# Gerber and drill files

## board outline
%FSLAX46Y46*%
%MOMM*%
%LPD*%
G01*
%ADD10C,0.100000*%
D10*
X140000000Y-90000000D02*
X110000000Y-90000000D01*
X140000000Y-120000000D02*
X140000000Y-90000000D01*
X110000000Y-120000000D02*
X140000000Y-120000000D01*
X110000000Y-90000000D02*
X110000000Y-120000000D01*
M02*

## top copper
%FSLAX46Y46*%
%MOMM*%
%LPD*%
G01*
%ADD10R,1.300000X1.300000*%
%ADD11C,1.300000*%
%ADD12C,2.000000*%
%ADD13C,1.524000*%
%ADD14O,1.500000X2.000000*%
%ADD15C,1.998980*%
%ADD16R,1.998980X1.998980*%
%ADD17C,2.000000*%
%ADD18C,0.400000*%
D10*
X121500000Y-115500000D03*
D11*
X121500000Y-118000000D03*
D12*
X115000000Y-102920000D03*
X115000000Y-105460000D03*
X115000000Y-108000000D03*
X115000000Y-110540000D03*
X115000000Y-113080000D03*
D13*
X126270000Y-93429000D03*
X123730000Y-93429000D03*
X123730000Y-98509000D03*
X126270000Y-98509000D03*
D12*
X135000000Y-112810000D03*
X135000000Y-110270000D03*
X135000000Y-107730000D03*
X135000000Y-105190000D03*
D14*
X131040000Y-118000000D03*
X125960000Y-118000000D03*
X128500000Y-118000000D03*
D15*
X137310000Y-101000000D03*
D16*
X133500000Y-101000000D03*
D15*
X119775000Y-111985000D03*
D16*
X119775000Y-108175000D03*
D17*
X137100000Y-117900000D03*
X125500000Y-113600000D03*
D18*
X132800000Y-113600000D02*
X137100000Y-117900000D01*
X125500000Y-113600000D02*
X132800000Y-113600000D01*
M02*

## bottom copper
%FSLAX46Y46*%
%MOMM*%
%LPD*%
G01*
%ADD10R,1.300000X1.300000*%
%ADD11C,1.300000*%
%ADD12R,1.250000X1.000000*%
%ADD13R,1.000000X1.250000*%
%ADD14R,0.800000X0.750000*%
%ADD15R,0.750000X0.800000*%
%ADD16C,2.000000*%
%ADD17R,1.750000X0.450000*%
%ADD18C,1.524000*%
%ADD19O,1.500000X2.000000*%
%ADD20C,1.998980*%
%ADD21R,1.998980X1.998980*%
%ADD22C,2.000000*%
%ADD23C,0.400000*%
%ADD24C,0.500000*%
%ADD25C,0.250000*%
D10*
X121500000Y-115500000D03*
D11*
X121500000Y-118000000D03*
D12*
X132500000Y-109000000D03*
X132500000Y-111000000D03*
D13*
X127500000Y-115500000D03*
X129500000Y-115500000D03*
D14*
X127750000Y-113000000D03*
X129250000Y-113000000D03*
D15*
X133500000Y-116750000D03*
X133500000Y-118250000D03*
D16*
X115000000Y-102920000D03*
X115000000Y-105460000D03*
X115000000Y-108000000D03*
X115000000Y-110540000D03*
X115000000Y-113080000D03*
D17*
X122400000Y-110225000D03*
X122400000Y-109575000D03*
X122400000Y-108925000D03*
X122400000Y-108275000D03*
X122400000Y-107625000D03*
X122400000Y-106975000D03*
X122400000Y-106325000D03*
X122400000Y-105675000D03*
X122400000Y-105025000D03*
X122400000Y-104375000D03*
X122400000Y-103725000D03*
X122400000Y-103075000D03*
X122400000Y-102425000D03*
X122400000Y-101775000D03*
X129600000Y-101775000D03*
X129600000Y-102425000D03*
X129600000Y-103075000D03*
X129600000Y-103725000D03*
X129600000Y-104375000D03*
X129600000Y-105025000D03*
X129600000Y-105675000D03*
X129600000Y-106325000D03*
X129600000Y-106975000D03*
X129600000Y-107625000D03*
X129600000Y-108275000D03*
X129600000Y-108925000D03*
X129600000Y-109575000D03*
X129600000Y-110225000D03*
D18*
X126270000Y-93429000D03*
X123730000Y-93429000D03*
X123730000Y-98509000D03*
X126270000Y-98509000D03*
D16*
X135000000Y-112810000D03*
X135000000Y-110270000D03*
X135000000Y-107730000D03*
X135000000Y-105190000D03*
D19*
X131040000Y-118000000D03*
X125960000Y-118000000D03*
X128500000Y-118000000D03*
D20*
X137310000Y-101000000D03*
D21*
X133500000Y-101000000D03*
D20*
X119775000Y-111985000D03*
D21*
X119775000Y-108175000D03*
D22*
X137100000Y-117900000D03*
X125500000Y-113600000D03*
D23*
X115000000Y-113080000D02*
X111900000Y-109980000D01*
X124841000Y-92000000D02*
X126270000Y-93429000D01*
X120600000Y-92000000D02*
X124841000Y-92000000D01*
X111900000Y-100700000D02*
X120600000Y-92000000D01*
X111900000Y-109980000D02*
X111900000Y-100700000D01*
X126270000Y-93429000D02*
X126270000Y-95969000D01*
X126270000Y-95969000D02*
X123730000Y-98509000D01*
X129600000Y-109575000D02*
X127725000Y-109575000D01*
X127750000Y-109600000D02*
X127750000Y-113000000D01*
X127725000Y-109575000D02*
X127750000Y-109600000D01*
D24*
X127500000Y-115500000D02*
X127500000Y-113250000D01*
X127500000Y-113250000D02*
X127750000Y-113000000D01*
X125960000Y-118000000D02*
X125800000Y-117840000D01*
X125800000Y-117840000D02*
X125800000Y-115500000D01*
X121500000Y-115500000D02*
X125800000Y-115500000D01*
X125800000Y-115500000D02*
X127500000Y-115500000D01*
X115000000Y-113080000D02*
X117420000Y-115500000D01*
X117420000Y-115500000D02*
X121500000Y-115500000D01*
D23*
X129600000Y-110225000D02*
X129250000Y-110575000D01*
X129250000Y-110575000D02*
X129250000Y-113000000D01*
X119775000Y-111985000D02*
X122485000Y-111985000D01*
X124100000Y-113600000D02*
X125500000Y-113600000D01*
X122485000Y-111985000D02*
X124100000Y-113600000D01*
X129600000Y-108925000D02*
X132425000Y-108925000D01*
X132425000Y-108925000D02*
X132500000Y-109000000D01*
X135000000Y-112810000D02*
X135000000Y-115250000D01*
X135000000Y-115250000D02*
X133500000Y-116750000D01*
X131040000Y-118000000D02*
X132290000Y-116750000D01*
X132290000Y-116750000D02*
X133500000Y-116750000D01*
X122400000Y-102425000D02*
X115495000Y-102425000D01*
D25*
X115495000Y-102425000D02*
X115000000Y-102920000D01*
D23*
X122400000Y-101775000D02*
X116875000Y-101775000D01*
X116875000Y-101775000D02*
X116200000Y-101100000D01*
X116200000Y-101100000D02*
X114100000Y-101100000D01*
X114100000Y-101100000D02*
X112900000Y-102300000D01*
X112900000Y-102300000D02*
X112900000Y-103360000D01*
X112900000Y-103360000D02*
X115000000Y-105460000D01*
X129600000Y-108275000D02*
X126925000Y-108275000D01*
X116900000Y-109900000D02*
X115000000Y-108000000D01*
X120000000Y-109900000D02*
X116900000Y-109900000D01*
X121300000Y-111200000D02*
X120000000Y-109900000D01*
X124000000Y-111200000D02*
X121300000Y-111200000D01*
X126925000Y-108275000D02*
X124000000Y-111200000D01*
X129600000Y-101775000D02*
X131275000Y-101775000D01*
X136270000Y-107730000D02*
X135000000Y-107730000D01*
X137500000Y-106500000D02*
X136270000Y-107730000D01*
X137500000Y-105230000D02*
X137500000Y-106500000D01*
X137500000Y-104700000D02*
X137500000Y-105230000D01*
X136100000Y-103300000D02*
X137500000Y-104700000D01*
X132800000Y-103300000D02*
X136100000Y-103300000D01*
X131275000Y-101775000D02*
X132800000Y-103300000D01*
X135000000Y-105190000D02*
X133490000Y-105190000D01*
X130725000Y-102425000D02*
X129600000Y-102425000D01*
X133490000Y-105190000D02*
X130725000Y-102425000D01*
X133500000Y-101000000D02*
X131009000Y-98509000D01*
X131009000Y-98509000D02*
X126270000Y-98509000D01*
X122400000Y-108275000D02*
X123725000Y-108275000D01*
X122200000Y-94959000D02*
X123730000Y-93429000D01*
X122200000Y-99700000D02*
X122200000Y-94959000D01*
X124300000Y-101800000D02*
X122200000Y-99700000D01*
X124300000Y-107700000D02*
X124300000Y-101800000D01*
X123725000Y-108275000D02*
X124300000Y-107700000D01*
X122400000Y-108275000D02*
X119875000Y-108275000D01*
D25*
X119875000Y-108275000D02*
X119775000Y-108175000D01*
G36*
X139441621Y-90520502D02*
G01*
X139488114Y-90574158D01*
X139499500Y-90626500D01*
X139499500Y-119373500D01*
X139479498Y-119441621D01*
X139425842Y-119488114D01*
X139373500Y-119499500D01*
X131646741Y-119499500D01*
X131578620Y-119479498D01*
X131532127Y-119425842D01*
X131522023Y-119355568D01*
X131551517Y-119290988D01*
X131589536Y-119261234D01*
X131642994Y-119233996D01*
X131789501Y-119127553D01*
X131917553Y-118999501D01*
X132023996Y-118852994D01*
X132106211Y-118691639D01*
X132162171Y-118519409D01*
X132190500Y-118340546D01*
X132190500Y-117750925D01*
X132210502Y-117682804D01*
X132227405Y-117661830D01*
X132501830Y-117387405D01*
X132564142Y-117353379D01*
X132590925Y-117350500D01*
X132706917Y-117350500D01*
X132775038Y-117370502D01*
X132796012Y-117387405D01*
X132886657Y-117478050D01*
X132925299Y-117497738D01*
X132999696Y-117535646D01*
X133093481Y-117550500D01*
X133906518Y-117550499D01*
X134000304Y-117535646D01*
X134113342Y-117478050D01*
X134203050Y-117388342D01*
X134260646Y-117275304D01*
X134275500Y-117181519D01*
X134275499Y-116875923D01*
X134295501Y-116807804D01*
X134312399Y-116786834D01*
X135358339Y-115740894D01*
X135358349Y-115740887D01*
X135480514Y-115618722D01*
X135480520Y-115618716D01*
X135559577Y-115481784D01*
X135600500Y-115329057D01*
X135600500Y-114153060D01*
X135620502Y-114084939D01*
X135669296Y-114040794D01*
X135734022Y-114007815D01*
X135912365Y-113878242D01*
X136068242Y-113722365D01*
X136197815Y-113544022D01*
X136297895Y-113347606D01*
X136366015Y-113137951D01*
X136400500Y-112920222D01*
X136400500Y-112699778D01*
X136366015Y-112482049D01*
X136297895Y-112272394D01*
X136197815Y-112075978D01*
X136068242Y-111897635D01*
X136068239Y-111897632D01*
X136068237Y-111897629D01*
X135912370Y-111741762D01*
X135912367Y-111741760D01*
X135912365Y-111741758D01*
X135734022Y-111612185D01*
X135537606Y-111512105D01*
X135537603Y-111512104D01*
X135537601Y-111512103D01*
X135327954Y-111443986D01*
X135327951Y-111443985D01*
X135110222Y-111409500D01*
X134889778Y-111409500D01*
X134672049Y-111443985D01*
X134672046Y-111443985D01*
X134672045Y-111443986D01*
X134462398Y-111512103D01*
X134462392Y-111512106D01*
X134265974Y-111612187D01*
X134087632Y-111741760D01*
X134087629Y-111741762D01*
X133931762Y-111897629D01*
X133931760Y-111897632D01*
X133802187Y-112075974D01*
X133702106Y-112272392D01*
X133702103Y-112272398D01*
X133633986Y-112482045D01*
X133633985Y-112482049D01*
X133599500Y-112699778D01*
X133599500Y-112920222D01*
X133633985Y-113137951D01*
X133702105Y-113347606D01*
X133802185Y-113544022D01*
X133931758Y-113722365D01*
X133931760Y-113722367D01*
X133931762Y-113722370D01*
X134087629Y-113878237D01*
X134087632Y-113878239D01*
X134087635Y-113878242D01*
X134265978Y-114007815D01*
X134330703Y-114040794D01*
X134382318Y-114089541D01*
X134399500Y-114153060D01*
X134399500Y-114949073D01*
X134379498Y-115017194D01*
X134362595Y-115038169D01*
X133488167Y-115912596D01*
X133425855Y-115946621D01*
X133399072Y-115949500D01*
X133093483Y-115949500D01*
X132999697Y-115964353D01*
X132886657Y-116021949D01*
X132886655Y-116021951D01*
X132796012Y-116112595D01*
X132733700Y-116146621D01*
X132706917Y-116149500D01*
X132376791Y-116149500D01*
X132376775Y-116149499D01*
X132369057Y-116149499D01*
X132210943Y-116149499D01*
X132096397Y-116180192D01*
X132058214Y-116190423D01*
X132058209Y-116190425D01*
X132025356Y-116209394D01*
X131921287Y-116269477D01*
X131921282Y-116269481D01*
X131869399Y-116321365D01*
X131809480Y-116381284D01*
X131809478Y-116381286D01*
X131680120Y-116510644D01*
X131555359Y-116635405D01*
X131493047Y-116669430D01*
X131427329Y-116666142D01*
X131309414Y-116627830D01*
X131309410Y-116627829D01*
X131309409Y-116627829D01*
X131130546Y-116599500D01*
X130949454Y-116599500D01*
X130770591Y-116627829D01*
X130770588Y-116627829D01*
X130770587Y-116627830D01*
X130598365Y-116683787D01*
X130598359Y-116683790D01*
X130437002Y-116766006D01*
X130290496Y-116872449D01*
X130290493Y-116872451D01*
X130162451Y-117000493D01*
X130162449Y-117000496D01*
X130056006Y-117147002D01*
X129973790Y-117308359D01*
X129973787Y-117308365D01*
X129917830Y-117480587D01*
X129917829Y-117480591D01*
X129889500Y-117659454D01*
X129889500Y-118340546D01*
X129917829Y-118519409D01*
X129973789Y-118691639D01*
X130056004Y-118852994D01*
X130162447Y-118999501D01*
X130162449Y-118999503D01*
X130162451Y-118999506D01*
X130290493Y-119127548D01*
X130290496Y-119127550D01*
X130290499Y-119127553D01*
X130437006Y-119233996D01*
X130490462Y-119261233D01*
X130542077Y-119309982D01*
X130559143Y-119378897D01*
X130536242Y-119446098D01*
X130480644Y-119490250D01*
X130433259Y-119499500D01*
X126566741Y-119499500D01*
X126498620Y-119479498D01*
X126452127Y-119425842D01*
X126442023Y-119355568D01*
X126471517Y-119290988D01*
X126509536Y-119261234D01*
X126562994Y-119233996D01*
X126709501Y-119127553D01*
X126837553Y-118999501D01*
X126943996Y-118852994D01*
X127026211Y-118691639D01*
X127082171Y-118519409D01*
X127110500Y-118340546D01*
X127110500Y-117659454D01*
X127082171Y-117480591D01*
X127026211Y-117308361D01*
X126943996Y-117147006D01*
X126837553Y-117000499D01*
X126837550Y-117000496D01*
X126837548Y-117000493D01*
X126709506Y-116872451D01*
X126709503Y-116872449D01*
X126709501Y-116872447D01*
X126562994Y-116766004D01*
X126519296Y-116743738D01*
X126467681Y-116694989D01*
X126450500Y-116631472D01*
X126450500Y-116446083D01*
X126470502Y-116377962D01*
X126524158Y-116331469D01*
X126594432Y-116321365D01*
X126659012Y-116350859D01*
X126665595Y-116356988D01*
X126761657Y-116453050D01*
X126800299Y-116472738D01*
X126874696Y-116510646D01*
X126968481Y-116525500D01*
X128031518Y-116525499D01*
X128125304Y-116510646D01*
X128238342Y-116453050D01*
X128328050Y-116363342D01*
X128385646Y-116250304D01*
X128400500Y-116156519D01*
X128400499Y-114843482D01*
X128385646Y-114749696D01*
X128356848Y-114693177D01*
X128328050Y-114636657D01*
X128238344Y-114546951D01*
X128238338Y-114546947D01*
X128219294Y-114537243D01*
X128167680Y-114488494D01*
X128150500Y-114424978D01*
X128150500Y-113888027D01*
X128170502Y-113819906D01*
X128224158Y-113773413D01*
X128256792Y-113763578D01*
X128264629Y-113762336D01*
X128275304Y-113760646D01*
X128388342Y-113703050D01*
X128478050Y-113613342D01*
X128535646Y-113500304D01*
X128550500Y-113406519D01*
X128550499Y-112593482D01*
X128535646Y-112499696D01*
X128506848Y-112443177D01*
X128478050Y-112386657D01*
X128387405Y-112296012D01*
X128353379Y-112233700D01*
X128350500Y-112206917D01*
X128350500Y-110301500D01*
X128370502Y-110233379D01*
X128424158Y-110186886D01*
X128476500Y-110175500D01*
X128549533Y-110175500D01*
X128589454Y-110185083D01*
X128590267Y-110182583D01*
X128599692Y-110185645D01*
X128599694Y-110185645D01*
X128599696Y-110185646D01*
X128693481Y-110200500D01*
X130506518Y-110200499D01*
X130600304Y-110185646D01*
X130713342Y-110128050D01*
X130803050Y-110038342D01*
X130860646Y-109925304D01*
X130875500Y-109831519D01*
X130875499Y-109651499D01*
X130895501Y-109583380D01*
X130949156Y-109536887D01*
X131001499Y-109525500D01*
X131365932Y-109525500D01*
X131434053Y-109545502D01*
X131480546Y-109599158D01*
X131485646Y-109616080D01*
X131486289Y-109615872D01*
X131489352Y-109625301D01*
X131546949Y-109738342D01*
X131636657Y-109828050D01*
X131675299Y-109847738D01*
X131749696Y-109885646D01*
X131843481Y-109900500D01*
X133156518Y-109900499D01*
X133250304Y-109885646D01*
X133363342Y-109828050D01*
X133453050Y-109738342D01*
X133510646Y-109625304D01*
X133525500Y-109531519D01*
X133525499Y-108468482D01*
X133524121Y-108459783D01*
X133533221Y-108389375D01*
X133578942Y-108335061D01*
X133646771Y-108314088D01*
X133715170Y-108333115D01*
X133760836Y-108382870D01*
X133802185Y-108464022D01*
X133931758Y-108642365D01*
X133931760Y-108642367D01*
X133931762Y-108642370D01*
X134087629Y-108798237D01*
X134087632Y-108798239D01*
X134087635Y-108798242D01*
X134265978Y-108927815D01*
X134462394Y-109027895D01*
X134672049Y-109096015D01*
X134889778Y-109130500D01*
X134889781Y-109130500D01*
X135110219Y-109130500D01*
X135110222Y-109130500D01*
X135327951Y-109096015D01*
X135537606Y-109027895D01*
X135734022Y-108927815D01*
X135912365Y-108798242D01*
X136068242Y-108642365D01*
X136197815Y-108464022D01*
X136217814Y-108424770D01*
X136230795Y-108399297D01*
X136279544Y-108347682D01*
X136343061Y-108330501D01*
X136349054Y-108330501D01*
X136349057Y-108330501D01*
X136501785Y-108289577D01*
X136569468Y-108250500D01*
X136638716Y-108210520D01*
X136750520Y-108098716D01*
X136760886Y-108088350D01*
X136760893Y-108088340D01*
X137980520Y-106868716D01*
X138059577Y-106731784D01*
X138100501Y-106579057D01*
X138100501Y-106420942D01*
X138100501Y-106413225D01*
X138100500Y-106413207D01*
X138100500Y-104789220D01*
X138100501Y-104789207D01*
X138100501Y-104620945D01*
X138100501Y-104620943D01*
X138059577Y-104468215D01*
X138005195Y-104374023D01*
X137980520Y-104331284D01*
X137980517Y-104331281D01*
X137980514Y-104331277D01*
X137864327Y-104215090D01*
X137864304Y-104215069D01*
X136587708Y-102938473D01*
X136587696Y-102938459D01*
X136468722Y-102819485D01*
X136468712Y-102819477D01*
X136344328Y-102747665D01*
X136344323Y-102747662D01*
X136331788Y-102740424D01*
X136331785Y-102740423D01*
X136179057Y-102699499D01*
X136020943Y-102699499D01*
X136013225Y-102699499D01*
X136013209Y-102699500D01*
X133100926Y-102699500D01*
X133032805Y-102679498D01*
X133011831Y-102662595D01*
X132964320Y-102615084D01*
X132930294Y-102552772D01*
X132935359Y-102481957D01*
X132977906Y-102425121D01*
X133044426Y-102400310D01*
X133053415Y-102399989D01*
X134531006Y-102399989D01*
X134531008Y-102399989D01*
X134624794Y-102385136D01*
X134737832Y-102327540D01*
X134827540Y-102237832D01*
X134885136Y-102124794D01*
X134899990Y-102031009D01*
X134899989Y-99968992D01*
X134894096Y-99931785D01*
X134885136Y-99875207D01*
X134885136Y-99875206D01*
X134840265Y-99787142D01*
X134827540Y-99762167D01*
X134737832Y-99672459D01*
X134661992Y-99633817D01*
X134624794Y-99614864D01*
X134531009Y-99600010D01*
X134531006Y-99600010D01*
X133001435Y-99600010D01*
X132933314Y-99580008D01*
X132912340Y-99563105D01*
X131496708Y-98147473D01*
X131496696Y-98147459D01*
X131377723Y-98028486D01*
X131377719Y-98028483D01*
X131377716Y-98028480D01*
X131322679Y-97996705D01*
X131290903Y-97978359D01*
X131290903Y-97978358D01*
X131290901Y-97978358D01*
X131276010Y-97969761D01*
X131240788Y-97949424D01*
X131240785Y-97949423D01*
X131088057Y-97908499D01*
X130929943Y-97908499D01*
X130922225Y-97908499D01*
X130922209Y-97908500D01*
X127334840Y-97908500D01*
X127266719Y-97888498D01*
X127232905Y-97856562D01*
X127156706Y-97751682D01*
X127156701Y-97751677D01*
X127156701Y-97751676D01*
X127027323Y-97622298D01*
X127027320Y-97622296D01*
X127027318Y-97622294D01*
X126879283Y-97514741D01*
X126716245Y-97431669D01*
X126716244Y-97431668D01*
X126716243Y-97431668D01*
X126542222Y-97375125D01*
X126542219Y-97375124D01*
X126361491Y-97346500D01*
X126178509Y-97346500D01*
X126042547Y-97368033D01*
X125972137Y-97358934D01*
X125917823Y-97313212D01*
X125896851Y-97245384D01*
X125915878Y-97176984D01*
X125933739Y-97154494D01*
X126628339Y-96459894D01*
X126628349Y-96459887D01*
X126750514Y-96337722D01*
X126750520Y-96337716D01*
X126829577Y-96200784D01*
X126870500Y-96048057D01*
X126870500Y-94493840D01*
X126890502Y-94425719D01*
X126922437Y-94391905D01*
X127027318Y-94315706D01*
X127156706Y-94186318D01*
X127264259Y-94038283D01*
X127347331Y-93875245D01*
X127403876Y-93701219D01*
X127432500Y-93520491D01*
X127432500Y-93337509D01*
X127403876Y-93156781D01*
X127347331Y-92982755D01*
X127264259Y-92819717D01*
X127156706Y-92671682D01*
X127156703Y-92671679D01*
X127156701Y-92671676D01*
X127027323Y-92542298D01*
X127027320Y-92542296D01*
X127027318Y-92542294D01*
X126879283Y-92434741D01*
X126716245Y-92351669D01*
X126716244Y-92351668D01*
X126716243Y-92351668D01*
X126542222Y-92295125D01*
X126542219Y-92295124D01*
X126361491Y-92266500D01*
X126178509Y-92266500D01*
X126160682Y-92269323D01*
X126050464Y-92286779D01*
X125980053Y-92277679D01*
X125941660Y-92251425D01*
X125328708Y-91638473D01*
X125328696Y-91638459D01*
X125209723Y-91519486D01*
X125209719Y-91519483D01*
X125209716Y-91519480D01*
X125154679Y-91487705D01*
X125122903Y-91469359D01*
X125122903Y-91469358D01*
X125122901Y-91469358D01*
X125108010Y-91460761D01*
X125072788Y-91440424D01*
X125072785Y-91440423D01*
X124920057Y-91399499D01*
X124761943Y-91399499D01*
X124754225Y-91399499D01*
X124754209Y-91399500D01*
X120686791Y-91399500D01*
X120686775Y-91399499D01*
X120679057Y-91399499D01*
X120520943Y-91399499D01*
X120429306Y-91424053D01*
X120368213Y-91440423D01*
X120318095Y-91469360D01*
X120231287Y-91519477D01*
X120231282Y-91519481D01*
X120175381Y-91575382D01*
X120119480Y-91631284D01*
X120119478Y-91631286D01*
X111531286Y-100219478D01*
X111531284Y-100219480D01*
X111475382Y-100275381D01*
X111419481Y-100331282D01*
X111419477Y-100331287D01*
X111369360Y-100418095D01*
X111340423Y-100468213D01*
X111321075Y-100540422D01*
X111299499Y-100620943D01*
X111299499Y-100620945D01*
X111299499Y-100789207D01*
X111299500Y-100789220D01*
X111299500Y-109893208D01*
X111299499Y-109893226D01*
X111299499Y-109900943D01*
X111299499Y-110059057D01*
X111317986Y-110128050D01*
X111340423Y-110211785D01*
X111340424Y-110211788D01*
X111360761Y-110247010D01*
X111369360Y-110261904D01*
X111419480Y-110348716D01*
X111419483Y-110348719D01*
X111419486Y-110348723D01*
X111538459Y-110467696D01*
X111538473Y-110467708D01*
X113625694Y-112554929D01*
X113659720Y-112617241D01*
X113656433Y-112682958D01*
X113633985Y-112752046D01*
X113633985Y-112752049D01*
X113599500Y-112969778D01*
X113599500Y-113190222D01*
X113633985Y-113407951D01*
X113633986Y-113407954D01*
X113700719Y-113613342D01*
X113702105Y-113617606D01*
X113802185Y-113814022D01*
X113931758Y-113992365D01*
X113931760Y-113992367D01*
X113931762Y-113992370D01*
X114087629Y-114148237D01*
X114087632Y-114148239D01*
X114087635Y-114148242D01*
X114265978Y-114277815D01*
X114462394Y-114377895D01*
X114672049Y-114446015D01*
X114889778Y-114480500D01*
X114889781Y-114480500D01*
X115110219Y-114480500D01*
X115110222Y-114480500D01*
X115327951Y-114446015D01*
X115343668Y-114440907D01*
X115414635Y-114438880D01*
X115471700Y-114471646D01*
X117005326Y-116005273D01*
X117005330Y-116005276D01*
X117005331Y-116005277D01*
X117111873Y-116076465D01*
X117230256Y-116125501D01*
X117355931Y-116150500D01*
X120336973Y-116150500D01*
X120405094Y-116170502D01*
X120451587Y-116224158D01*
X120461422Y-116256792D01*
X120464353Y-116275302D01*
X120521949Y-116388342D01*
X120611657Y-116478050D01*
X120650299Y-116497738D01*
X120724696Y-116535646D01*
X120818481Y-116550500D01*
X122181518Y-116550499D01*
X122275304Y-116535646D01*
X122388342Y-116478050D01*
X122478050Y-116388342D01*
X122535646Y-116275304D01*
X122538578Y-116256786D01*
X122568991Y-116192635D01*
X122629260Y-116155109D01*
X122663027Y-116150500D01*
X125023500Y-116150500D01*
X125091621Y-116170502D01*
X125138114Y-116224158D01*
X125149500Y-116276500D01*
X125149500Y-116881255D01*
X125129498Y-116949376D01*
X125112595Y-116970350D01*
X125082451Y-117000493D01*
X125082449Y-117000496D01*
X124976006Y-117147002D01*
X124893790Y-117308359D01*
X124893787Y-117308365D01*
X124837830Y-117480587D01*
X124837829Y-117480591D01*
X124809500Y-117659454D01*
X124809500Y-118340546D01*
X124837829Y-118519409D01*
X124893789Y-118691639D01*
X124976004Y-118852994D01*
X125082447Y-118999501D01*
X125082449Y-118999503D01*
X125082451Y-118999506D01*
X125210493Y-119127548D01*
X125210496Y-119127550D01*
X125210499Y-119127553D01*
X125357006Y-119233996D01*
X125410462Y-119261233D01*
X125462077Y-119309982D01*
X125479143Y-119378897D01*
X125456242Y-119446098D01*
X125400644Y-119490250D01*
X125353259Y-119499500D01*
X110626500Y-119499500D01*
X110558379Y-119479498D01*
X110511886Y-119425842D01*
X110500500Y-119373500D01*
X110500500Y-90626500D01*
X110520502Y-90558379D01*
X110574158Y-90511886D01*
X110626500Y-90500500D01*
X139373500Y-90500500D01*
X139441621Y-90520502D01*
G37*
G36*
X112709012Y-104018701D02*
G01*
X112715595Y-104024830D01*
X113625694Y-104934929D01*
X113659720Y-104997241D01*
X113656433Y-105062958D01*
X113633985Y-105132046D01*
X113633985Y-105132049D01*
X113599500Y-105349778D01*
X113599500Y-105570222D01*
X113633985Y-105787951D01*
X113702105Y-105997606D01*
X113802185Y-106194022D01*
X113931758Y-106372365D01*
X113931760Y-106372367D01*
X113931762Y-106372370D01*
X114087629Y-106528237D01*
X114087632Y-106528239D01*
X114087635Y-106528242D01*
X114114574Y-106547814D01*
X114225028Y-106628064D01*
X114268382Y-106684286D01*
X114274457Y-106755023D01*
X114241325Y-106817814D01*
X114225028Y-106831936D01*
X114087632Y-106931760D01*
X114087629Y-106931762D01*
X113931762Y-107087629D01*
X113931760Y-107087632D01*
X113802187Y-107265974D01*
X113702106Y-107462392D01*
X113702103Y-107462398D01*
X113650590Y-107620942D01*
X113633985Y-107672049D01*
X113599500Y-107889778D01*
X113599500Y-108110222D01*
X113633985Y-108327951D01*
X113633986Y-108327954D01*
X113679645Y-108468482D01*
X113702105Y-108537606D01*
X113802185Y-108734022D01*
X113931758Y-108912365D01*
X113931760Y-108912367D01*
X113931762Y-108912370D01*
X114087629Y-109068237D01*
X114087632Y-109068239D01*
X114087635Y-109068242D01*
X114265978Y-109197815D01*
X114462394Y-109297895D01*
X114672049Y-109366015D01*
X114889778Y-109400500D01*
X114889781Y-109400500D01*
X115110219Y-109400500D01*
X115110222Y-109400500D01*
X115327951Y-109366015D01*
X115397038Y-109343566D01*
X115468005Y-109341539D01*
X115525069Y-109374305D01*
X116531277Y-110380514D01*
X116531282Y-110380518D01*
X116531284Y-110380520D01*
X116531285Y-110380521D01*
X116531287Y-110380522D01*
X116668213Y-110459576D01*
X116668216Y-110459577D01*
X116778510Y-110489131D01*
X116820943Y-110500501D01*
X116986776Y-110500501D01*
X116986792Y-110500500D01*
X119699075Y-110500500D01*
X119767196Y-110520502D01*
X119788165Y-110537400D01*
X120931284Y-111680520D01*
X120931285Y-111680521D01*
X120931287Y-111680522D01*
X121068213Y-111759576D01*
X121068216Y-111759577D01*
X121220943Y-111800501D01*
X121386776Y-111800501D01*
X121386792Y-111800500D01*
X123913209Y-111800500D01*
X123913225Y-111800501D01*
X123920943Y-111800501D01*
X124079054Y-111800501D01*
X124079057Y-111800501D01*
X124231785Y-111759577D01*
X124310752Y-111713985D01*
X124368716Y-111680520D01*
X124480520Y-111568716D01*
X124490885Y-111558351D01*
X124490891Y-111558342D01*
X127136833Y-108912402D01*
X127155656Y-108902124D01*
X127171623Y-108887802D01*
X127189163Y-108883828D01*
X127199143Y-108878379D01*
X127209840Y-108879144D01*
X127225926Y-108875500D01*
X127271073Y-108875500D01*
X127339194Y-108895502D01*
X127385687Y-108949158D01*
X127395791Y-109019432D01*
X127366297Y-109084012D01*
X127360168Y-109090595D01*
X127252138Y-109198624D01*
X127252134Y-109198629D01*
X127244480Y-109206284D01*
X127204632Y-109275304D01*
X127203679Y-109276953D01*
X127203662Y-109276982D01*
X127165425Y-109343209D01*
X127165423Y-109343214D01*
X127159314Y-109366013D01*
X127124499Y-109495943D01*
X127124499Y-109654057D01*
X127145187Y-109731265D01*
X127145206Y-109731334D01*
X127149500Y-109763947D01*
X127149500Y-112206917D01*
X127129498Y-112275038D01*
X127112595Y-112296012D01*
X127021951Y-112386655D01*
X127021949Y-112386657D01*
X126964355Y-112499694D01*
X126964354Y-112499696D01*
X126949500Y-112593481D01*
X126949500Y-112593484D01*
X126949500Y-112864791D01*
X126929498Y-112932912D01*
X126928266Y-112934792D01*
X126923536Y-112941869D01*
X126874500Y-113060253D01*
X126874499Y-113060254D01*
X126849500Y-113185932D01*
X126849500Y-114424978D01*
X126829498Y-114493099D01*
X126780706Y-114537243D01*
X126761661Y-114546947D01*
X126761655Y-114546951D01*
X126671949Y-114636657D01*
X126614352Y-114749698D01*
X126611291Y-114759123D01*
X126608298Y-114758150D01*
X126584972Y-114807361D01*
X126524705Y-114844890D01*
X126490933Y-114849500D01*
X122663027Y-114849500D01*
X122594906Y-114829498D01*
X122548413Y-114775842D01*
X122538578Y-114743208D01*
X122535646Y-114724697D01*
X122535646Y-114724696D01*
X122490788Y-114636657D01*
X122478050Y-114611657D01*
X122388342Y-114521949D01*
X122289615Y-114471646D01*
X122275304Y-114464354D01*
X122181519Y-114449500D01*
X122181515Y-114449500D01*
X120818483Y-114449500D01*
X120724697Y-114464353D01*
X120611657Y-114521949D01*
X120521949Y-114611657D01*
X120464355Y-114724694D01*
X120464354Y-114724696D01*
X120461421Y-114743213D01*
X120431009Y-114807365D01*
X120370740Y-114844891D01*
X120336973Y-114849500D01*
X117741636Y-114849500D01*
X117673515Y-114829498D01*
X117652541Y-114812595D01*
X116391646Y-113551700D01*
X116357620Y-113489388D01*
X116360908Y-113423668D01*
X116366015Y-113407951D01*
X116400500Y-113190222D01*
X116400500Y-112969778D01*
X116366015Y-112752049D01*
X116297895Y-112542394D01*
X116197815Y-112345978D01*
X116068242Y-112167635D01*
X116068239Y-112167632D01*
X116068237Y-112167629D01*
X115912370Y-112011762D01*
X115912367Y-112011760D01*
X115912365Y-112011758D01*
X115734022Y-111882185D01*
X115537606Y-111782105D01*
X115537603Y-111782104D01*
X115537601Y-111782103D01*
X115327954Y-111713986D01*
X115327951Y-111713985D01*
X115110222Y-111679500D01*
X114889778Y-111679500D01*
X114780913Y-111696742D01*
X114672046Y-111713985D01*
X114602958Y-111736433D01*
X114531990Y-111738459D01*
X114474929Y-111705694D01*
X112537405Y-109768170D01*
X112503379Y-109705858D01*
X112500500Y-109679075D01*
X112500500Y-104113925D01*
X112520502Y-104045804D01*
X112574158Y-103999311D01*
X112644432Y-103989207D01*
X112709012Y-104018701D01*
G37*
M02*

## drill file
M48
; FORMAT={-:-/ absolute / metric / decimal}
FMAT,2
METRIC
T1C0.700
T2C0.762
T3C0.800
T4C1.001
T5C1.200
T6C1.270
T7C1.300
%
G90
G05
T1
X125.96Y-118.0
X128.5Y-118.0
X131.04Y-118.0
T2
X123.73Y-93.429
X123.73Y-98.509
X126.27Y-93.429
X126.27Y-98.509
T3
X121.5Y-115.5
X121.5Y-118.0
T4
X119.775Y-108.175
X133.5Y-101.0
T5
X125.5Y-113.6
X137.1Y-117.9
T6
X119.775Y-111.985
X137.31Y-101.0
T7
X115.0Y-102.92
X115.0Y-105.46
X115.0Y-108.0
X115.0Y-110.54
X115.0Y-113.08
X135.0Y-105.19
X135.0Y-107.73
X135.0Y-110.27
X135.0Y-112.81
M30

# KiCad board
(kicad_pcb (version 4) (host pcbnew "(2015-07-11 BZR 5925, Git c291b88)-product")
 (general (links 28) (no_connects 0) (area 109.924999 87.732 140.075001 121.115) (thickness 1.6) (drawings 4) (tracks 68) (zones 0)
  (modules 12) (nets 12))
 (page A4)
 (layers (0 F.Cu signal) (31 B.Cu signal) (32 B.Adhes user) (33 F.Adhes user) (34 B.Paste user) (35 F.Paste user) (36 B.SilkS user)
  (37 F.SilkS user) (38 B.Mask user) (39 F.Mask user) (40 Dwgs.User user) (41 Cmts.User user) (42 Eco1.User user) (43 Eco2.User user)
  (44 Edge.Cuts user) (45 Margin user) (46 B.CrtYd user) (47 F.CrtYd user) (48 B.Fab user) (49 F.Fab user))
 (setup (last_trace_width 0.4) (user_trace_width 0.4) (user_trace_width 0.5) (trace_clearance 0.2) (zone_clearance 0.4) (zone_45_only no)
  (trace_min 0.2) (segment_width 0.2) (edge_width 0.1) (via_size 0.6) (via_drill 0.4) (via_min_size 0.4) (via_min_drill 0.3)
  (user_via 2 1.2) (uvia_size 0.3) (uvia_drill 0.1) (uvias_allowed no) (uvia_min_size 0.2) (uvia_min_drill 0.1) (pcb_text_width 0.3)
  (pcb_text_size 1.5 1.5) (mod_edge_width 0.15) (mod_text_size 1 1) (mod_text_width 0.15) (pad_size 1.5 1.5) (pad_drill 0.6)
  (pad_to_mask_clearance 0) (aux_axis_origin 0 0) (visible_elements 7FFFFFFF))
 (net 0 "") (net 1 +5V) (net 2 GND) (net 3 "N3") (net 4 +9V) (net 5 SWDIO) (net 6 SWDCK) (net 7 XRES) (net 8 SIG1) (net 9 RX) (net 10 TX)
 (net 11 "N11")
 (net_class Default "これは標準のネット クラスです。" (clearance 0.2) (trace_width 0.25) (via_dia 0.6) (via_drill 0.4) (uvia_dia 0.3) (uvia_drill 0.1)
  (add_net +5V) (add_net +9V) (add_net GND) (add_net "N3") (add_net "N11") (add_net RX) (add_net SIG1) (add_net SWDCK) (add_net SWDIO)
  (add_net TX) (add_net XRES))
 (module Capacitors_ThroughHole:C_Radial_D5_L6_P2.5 (layer F.Cu) (at 121.5 115.5 270)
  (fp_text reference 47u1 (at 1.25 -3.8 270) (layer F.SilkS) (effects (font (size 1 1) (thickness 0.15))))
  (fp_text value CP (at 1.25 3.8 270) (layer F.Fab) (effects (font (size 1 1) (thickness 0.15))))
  (pad 1 thru_hole rect (at 0 0 270) (size 1.3 1.3) (drill 0.8) (layers *.Cu *.Mask F.SilkS) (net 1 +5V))
  (pad 2 thru_hole circle (at 2.5 0 270) (size 1.3 1.3) (drill 0.8) (layers *.Cu *.Mask F.SilkS) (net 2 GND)))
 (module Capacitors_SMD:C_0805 (layer B.Cu) (at 132.5 110 270)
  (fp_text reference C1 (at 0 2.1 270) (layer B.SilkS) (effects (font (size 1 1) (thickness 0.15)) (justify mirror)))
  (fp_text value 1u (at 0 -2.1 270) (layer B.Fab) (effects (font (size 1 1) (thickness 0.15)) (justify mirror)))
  (pad 1 smd rect (at -1 0 270) (size 1 1.25) (layers B.Cu B.Paste B.Mask) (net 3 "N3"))
  (pad 2 smd rect (at 1 0 270) (size 1 1.25) (layers B.Cu B.Paste B.Mask) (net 2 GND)))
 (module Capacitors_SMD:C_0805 (layer B.Cu) (at 128.5 115.5)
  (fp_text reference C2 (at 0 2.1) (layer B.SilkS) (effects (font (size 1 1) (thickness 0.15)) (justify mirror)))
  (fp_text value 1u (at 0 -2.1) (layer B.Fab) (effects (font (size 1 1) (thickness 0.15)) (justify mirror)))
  (pad 1 smd rect (at -1 0) (size 1 1.25) (layers B.Cu B.Paste B.Mask) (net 1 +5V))
  (pad 2 smd rect (at 1 0) (size 1 1.25) (layers B.Cu B.Paste B.Mask) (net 2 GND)))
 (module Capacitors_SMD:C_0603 (layer B.Cu) (at 128.5 113)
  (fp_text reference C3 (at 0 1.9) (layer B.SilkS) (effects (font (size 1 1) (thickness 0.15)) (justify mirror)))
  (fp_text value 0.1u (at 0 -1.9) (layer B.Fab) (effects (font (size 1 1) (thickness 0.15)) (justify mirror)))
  (pad 1 smd rect (at -0.75 0) (size 0.8 0.75) (layers B.Cu B.Paste B.Mask) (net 1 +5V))
  (pad 2 smd rect (at 0.75 0) (size 0.8 0.75) (layers B.Cu B.Paste B.Mask) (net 2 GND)))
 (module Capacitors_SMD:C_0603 (layer B.Cu) (at 133.5 117.5 270)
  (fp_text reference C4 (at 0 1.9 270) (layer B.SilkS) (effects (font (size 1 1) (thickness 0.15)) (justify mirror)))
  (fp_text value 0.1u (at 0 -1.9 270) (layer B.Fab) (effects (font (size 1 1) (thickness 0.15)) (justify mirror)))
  (pad 1 smd rect (at -0.75 0 270) (size 0.8 0.75) (layers B.Cu B.Paste B.Mask) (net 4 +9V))
  (pad 2 smd rect (at 0.75 0 270) (size 0.8 0.75) (layers B.Cu B.Paste B.Mask) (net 2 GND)))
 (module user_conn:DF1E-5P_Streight (layer F.Cu) (at 115 108 270)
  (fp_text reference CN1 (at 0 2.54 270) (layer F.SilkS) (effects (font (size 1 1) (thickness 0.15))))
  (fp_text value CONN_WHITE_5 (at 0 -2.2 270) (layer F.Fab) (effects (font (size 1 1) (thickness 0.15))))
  (pad 1 thru_hole circle (at -5.08 0 270) (size 2 2) (drill 1.3) (layers *.Cu *.Mask F.SilkS) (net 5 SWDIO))
  (pad 2 thru_hole circle (at -2.54 0 270) (size 2 2) (drill 1.3) (layers *.Cu *.Mask F.SilkS) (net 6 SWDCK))
  (pad 3 thru_hole circle (at 0 0 270) (size 2 2) (drill 1.3) (layers *.Cu *.Mask F.SilkS) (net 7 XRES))
  (pad 4 thru_hole circle (at 2.54 0 270) (size 2 2) (drill 1.3) (layers *.Cu *.Mask F.SilkS) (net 2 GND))
  (pad 5 thru_hole circle (at 5.08 0 270) (size 2 2) (drill 1.3) (layers *.Cu *.Mask F.SilkS) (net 1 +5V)))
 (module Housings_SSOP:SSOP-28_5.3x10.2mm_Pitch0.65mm (layer B.Cu) (at 126 106)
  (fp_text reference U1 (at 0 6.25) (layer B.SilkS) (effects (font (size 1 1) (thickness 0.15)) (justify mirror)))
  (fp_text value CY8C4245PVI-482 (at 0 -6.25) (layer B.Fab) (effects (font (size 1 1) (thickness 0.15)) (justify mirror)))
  (pad 1 smd rect (at -3.6 4.225) (size 1.75 0.45) (layers B.Cu B.Paste B.Mask))
  (pad 2 smd rect (at -3.6 3.575) (size 1.75 0.45) (layers B.Cu B.Paste B.Mask))
  (pad 3 smd rect (at -3.6 2.925) (size 1.75 0.45) (layers B.Cu B.Paste B.Mask))
  (pad 4 smd rect (at -3.6 2.275) (size 1.75 0.45) (layers B.Cu B.Paste B.Mask) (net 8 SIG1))
  (pad 5 smd rect (at -3.6 1.625) (size 1.75 0.45) (layers B.Cu B.Paste B.Mask))
  (pad 6 smd rect (at -3.6 0.975) (size 1.75 0.45) (layers B.Cu B.Paste B.Mask))
  (pad 7 smd rect (at -3.6 0.325) (size 1.75 0.45) (layers B.Cu B.Paste B.Mask))
  (pad 8 smd rect (at -3.6 -0.325) (size 1.75 0.45) (layers B.Cu B.Paste B.Mask))
  (pad 9 smd rect (at -3.6 -0.975) (size 1.75 0.45) (layers B.Cu B.Paste B.Mask))
  (pad 10 smd rect (at -3.6 -1.625) (size 1.75 0.45) (layers B.Cu B.Paste B.Mask))
  (pad 11 smd rect (at -3.6 -2.275) (size 1.75 0.45) (layers B.Cu B.Paste B.Mask))
  (pad 12 smd rect (at -3.6 -2.925) (size 1.75 0.45) (layers B.Cu B.Paste B.Mask))
  (pad 13 smd rect (at -3.6 -3.575) (size 1.75 0.45) (layers B.Cu B.Paste B.Mask) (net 5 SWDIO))
  (pad 14 smd rect (at -3.6 -4.225) (size 1.75 0.45) (layers B.Cu B.Paste B.Mask) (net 6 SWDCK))
  (pad 15 smd rect (at 3.6 -4.225) (size 1.75 0.45) (layers B.Cu B.Paste B.Mask) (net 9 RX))
  (pad 16 smd rect (at 3.6 -3.575) (size 1.75 0.45) (layers B.Cu B.Paste B.Mask) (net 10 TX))
  (pad 17 smd rect (at 3.6 -2.925) (size 1.75 0.45) (layers B.Cu B.Paste B.Mask))
  (pad 18 smd rect (at 3.6 -2.275) (size 1.75 0.45) (layers B.Cu B.Paste B.Mask))
  (pad 19 smd rect (at 3.6 -1.625) (size 1.75 0.45) (layers B.Cu B.Paste B.Mask))
  (pad 20 smd rect (at 3.6 -0.975) (size 1.75 0.45) (layers B.Cu B.Paste B.Mask))
  (pad 21 smd rect (at 3.6 -0.325) (size 1.75 0.45) (layers B.Cu B.Paste B.Mask))
  (pad 22 smd rect (at 3.6 0.325) (size 1.75 0.45) (layers B.Cu B.Paste B.Mask))
  (pad 23 smd rect (at 3.6 0.975) (size 1.75 0.45) (layers B.Cu B.Paste B.Mask))
  (pad 24 smd rect (at 3.6 1.625) (size 1.75 0.45) (layers B.Cu B.Paste B.Mask))
  (pad 25 smd rect (at 3.6 2.275) (size 1.75 0.45) (layers B.Cu B.Paste B.Mask) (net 7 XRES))
  (pad 26 smd rect (at 3.6 2.925) (size 1.75 0.45) (layers B.Cu B.Paste B.Mask) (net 3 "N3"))
  (pad 27 smd rect (at 3.6 3.575) (size 1.75 0.45) (layers B.Cu B.Paste B.Mask) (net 1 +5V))
  (pad 28 smd rect (at 3.6 4.225) (size 1.75 0.45) (layers B.Cu B.Paste B.Mask) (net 2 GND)))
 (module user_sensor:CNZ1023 (layer F.Cu) (at 125 90 180)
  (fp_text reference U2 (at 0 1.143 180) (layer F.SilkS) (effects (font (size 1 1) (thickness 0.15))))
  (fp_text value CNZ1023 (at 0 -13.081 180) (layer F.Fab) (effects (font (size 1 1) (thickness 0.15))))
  (pad 3 thru_hole circle (at -1.27 -3.429 180) (size 1.524 1.524) (drill 0.762) (layers *.Cu *.Mask F.SilkS) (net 1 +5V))
  (pad 4 thru_hole circle (at 1.27 -3.429 180) (size 1.524 1.524) (drill 0.762) (layers *.Cu *.Mask F.SilkS) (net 8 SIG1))
  (pad 1 thru_hole circle (at 1.27 -8.509 180) (size 1.524 1.524) (drill 0.762) (layers *.Cu *.Mask F.SilkS) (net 1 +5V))
  (pad 2 thru_hole circle (at -1.27 -8.509 180) (size 1.524 1.524) (drill 0.762) (layers *.Cu *.Mask F.SilkS) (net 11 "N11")))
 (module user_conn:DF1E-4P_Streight (layer F.Cu) (at 135 109 90)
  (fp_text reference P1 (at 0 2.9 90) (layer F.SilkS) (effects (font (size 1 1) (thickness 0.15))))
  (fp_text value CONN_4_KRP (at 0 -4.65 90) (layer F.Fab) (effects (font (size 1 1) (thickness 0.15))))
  (pad 1 thru_hole circle (at -3.81 0 90) (size 2 2) (drill 1.3) (layers *.Cu *.Mask F.SilkS) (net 4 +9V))
  (pad 2 thru_hole circle (at -1.27 0 90) (size 2 2) (drill 1.3) (layers *.Cu *.Mask F.SilkS) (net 2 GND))
  (pad 3 thru_hole circle (at 1.27 0 90) (size 2 2) (drill 1.3) (layers *.Cu *.Mask F.SilkS) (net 9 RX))
  (pad 4 thru_hole circle (at 3.81 0 90) (size 2 2) (drill 1.3) (layers *.Cu *.Mask F.SilkS) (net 10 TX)))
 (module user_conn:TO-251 (layer F.Cu) (at 128.5 118 180)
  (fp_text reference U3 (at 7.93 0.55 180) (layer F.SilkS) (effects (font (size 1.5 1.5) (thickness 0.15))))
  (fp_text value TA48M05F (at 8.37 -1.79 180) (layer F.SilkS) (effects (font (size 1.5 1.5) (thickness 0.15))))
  (pad 1 thru_hole oval (at -2.54 0 180) (size 1.5 2) (drill 0.7) (layers *.Cu *.Mask F.SilkS) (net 4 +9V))
  (pad 2 thru_hole oval (at 2.54 0 180) (size 1.5 2) (drill 0.7) (layers *.Cu *.Mask F.SilkS) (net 1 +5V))
  (pad 3 thru_hole oval (at 0 0 180) (size 1.5 2) (drill 0.7) (layers *.Cu *.Mask F.SilkS) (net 2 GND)))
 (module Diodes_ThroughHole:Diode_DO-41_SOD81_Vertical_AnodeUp (layer F.Cu) (at 133.5 101)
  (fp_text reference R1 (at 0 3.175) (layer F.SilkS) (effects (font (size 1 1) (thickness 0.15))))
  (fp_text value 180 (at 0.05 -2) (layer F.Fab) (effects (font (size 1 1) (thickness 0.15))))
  (pad 2 thru_hole circle (at 3.81 0) (size 1.99898 1.99898) (drill 1.27) (layers *.Cu *.Mask F.SilkS) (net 2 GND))
  (pad 1 thru_hole rect (at 0 0) (size 1.99898 1.99898) (drill 1.00076) (layers *.Cu *.Mask F.SilkS) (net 11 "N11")))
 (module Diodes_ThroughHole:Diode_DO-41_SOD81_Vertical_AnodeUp (layer F.Cu) (at 119.775 108.175 270)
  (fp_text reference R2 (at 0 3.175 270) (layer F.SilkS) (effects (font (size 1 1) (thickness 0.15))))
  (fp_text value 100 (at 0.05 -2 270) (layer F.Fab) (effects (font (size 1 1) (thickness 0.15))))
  (pad 2 thru_hole circle (at 3.81 0 270) (size 1.99898 1.99898) (drill 1.27) (layers *.Cu *.Mask F.SilkS) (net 2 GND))
  (pad 1 thru_hole rect (at 0 0 270) (size 1.99898 1.99898) (drill 1.00076) (layers *.Cu *.Mask F.SilkS) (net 8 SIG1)))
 (gr_line (start 140 90) (end 110 90) (angle 90) (layer Edge.Cuts) (width 0.1))
 (gr_line (start 140 120) (end 140 90) (angle 90) (layer Edge.Cuts) (width 0.1))
 (gr_line (start 110 120) (end 140 120) (angle 90) (layer Edge.Cuts) (width 0.1))
 (gr_line (start 110 90) (end 110 120) (angle 90) (layer Edge.Cuts) (width 0.1))
 (segment (start 115 113.08) (end 111.9 109.98) (width 0.4) (layer B.Cu) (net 1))
 (segment (start 124.841 92) (end 126.27 93.429) (width 0.4) (layer B.Cu) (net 1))
 (segment (start 120.6 92) (end 124.841 92) (width 0.4) (layer B.Cu) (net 1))
 (segment (start 111.9 100.7) (end 120.6 92) (width 0.4) (layer B.Cu) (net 1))
 (segment (start 111.9 109.98) (end 111.9 100.7) (width 0.4) (layer B.Cu) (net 1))
 (segment (start 126.27 93.429) (end 126.27 95.969) (width 0.4) (layer B.Cu) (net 1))
 (segment (start 126.27 95.969) (end 123.73 98.509) (width 0.4) (layer B.Cu) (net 1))
 (segment (start 129.6 109.575) (end 127.725 109.575) (width 0.4) (layer B.Cu) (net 1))
 (segment (start 127.75 109.6) (end 127.75 113) (width 0.4) (layer B.Cu) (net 1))
 (segment (start 127.725 109.575) (end 127.75 109.6) (width 0.4) (layer B.Cu) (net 1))
 (segment (start 127.5 115.5) (end 127.5 113.25) (width 0.5) (layer B.Cu) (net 1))
 (segment (start 127.5 113.25) (end 127.75 113) (width 0.5) (layer B.Cu) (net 1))
 (segment (start 125.96 118) (end 125.8 117.84) (width 0.5) (layer B.Cu) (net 1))
 (segment (start 125.8 117.84) (end 125.8 115.5) (width 0.5) (layer B.Cu) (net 1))
 (segment (start 121.5 115.5) (end 125.8 115.5) (width 0.5) (layer B.Cu) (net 1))
 (segment (start 125.8 115.5) (end 127.5 115.5) (width 0.5) (layer B.Cu) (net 1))
 (segment (start 115 113.08) (end 117.42 115.5) (width 0.5) (layer B.Cu) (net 1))
 (segment (start 117.42 115.5) (end 121.5 115.5) (width 0.5) (layer B.Cu) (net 1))
 (segment (start 129.6 110.225) (end 129.25 110.575) (width 0.4) (layer B.Cu) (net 2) (status 400000))
 (segment (start 129.25 110.575) (end 129.25 113) (width 0.4) (layer B.Cu) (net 2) (status 800000))
 (segment (start 119.775 111.985) (end 122.485 111.985) (width 0.4) (layer B.Cu) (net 2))
 (via (at 137.1 117.9) (size 2) (drill 1.2) (layers F.Cu B.Cu) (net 2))
 (segment (start 132.8 113.6) (end 137.1 117.9) (width 0.4) (layer F.Cu) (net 2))
 (segment (start 125.5 113.6) (end 132.8 113.6) (width 0.4) (layer F.Cu) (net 2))
 (via (at 125.5 113.6) (size 2) (drill 1.2) (layers F.Cu B.Cu) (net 2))
 (segment (start 124.1 113.6) (end 125.5 113.6) (width 0.4) (layer B.Cu) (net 2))
 (segment (start 122.485 111.985) (end 124.1 113.6) (width 0.4) (layer B.Cu) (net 2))
 (segment (start 129.6 108.925) (end 132.425 108.925) (width 0.4) (layer B.Cu) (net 3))
 (segment (start 132.425 108.925) (end 132.5 109) (width 0.4) (layer B.Cu) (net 3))
 (segment (start 135 112.81) (end 135 115.25) (width 0.4) (layer B.Cu) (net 4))
 (segment (start 135 115.25) (end 133.5 116.75) (width 0.4) (layer B.Cu) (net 4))
 (segment (start 131.04 118) (end 132.29 116.75) (width 0.4) (layer B.Cu) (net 4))
 (segment (start 132.29 116.75) (end 133.5 116.75) (width 0.4) (layer B.Cu) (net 4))
 (segment (start 122.4 102.425) (end 115.495 102.425) (width 0.4) (layer B.Cu) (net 5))
 (segment (start 115.495 102.425) (end 115 102.92) (width 0.25) (layer B.Cu) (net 5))
 (segment (start 122.4 101.775) (end 116.875 101.775) (width 0.4) (layer B.Cu) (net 6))
 (segment (start 116.875 101.775) (end 116.2 101.1) (width 0.4) (layer B.Cu) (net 6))
 (segment (start 116.2 101.1) (end 114.1 101.1) (width 0.4) (layer B.Cu) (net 6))
 (segment (start 114.1 101.1) (end 112.9 102.3) (width 0.4) (layer B.Cu) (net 6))
 (segment (start 112.9 102.3) (end 112.9 103.36) (width 0.4) (layer B.Cu) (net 6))
 (segment (start 112.9 103.36) (end 115 105.46) (width 0.4) (layer B.Cu) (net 6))
 (segment (start 129.6 108.275) (end 126.925 108.275) (width 0.4) (layer B.Cu) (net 7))
 (segment (start 116.9 109.9) (end 115 108) (width 0.4) (layer B.Cu) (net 7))
 (segment (start 120 109.9) (end 116.9 109.9) (width 0.4) (layer B.Cu) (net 7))
 (segment (start 121.3 111.2) (end 120 109.9) (width 0.4) (layer B.Cu) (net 7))
 (segment (start 124 111.2) (end 121.3 111.2) (width 0.4) (layer B.Cu) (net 7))
 (segment (start 126.925 108.275) (end 124 111.2) (width 0.4) (layer B.Cu) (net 7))
 (segment (start 129.6 101.775) (end 131.275 101.775) (width 0.4) (layer B.Cu) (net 9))
 (segment (start 136.27 107.73) (end 135 107.73) (width 0.4) (layer B.Cu) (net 9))
 (segment (start 137.5 106.5) (end 136.27 107.73) (width 0.4) (layer B.Cu) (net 9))
 (segment (start 137.5 105.23) (end 137.5 106.5) (width 0.4) (layer B.Cu) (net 9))
 (segment (start 137.5 104.7) (end 137.5 105.23) (width 0.4) (layer B.Cu) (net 9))
 (segment (start 136.1 103.3) (end 137.5 104.7) (width 0.4) (layer B.Cu) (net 9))
 (segment (start 132.8 103.3) (end 136.1 103.3) (width 0.4) (layer B.Cu) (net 9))
 (segment (start 131.275 101.775) (end 132.8 103.3) (width 0.4) (layer B.Cu) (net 9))
 (segment (start 135 105.19) (end 133.49 105.19) (width 0.4) (layer B.Cu) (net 10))
 (segment (start 130.725 102.425) (end 129.6 102.425) (width 0.4) (layer B.Cu) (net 10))
 (segment (start 133.49 105.19) (end 130.725 102.425) (width 0.4) (layer B.Cu) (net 10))
 (segment (start 133.5 101) (end 131.009 98.509) (width 0.4) (layer B.Cu) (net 11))
 (segment (start 131.009 98.509) (end 126.27 98.509) (width 0.4) (layer B.Cu) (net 11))
 (segment (start 122.4 108.275) (end 123.725 108.275) (width 0.4) (layer B.Cu) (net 8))
 (segment (start 122.2 94.959) (end 123.73 93.429) (width 0.4) (layer B.Cu) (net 8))
 (segment (start 122.2 99.7) (end 122.2 94.959) (width 0.4) (layer B.Cu) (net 8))
 (segment (start 124.3 101.8) (end 122.2 99.7) (width 0.4) (layer B.Cu) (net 8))
 (segment (start 124.3 107.7) (end 124.3 101.8) (width 0.4) (layer B.Cu) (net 8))
 (segment (start 123.725 108.275) (end 124.3 107.7) (width 0.4) (layer B.Cu) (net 8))
 (segment (start 122.4 108.275) (end 119.875 108.275) (width 0.4) (layer B.Cu) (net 8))
 (segment (start 119.875 108.275) (end 119.775 108.175) (width 0.25) (layer B.Cu) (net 8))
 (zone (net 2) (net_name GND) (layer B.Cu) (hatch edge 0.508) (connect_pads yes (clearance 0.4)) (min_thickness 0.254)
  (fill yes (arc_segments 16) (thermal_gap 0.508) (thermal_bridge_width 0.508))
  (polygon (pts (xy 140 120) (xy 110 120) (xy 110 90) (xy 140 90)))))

